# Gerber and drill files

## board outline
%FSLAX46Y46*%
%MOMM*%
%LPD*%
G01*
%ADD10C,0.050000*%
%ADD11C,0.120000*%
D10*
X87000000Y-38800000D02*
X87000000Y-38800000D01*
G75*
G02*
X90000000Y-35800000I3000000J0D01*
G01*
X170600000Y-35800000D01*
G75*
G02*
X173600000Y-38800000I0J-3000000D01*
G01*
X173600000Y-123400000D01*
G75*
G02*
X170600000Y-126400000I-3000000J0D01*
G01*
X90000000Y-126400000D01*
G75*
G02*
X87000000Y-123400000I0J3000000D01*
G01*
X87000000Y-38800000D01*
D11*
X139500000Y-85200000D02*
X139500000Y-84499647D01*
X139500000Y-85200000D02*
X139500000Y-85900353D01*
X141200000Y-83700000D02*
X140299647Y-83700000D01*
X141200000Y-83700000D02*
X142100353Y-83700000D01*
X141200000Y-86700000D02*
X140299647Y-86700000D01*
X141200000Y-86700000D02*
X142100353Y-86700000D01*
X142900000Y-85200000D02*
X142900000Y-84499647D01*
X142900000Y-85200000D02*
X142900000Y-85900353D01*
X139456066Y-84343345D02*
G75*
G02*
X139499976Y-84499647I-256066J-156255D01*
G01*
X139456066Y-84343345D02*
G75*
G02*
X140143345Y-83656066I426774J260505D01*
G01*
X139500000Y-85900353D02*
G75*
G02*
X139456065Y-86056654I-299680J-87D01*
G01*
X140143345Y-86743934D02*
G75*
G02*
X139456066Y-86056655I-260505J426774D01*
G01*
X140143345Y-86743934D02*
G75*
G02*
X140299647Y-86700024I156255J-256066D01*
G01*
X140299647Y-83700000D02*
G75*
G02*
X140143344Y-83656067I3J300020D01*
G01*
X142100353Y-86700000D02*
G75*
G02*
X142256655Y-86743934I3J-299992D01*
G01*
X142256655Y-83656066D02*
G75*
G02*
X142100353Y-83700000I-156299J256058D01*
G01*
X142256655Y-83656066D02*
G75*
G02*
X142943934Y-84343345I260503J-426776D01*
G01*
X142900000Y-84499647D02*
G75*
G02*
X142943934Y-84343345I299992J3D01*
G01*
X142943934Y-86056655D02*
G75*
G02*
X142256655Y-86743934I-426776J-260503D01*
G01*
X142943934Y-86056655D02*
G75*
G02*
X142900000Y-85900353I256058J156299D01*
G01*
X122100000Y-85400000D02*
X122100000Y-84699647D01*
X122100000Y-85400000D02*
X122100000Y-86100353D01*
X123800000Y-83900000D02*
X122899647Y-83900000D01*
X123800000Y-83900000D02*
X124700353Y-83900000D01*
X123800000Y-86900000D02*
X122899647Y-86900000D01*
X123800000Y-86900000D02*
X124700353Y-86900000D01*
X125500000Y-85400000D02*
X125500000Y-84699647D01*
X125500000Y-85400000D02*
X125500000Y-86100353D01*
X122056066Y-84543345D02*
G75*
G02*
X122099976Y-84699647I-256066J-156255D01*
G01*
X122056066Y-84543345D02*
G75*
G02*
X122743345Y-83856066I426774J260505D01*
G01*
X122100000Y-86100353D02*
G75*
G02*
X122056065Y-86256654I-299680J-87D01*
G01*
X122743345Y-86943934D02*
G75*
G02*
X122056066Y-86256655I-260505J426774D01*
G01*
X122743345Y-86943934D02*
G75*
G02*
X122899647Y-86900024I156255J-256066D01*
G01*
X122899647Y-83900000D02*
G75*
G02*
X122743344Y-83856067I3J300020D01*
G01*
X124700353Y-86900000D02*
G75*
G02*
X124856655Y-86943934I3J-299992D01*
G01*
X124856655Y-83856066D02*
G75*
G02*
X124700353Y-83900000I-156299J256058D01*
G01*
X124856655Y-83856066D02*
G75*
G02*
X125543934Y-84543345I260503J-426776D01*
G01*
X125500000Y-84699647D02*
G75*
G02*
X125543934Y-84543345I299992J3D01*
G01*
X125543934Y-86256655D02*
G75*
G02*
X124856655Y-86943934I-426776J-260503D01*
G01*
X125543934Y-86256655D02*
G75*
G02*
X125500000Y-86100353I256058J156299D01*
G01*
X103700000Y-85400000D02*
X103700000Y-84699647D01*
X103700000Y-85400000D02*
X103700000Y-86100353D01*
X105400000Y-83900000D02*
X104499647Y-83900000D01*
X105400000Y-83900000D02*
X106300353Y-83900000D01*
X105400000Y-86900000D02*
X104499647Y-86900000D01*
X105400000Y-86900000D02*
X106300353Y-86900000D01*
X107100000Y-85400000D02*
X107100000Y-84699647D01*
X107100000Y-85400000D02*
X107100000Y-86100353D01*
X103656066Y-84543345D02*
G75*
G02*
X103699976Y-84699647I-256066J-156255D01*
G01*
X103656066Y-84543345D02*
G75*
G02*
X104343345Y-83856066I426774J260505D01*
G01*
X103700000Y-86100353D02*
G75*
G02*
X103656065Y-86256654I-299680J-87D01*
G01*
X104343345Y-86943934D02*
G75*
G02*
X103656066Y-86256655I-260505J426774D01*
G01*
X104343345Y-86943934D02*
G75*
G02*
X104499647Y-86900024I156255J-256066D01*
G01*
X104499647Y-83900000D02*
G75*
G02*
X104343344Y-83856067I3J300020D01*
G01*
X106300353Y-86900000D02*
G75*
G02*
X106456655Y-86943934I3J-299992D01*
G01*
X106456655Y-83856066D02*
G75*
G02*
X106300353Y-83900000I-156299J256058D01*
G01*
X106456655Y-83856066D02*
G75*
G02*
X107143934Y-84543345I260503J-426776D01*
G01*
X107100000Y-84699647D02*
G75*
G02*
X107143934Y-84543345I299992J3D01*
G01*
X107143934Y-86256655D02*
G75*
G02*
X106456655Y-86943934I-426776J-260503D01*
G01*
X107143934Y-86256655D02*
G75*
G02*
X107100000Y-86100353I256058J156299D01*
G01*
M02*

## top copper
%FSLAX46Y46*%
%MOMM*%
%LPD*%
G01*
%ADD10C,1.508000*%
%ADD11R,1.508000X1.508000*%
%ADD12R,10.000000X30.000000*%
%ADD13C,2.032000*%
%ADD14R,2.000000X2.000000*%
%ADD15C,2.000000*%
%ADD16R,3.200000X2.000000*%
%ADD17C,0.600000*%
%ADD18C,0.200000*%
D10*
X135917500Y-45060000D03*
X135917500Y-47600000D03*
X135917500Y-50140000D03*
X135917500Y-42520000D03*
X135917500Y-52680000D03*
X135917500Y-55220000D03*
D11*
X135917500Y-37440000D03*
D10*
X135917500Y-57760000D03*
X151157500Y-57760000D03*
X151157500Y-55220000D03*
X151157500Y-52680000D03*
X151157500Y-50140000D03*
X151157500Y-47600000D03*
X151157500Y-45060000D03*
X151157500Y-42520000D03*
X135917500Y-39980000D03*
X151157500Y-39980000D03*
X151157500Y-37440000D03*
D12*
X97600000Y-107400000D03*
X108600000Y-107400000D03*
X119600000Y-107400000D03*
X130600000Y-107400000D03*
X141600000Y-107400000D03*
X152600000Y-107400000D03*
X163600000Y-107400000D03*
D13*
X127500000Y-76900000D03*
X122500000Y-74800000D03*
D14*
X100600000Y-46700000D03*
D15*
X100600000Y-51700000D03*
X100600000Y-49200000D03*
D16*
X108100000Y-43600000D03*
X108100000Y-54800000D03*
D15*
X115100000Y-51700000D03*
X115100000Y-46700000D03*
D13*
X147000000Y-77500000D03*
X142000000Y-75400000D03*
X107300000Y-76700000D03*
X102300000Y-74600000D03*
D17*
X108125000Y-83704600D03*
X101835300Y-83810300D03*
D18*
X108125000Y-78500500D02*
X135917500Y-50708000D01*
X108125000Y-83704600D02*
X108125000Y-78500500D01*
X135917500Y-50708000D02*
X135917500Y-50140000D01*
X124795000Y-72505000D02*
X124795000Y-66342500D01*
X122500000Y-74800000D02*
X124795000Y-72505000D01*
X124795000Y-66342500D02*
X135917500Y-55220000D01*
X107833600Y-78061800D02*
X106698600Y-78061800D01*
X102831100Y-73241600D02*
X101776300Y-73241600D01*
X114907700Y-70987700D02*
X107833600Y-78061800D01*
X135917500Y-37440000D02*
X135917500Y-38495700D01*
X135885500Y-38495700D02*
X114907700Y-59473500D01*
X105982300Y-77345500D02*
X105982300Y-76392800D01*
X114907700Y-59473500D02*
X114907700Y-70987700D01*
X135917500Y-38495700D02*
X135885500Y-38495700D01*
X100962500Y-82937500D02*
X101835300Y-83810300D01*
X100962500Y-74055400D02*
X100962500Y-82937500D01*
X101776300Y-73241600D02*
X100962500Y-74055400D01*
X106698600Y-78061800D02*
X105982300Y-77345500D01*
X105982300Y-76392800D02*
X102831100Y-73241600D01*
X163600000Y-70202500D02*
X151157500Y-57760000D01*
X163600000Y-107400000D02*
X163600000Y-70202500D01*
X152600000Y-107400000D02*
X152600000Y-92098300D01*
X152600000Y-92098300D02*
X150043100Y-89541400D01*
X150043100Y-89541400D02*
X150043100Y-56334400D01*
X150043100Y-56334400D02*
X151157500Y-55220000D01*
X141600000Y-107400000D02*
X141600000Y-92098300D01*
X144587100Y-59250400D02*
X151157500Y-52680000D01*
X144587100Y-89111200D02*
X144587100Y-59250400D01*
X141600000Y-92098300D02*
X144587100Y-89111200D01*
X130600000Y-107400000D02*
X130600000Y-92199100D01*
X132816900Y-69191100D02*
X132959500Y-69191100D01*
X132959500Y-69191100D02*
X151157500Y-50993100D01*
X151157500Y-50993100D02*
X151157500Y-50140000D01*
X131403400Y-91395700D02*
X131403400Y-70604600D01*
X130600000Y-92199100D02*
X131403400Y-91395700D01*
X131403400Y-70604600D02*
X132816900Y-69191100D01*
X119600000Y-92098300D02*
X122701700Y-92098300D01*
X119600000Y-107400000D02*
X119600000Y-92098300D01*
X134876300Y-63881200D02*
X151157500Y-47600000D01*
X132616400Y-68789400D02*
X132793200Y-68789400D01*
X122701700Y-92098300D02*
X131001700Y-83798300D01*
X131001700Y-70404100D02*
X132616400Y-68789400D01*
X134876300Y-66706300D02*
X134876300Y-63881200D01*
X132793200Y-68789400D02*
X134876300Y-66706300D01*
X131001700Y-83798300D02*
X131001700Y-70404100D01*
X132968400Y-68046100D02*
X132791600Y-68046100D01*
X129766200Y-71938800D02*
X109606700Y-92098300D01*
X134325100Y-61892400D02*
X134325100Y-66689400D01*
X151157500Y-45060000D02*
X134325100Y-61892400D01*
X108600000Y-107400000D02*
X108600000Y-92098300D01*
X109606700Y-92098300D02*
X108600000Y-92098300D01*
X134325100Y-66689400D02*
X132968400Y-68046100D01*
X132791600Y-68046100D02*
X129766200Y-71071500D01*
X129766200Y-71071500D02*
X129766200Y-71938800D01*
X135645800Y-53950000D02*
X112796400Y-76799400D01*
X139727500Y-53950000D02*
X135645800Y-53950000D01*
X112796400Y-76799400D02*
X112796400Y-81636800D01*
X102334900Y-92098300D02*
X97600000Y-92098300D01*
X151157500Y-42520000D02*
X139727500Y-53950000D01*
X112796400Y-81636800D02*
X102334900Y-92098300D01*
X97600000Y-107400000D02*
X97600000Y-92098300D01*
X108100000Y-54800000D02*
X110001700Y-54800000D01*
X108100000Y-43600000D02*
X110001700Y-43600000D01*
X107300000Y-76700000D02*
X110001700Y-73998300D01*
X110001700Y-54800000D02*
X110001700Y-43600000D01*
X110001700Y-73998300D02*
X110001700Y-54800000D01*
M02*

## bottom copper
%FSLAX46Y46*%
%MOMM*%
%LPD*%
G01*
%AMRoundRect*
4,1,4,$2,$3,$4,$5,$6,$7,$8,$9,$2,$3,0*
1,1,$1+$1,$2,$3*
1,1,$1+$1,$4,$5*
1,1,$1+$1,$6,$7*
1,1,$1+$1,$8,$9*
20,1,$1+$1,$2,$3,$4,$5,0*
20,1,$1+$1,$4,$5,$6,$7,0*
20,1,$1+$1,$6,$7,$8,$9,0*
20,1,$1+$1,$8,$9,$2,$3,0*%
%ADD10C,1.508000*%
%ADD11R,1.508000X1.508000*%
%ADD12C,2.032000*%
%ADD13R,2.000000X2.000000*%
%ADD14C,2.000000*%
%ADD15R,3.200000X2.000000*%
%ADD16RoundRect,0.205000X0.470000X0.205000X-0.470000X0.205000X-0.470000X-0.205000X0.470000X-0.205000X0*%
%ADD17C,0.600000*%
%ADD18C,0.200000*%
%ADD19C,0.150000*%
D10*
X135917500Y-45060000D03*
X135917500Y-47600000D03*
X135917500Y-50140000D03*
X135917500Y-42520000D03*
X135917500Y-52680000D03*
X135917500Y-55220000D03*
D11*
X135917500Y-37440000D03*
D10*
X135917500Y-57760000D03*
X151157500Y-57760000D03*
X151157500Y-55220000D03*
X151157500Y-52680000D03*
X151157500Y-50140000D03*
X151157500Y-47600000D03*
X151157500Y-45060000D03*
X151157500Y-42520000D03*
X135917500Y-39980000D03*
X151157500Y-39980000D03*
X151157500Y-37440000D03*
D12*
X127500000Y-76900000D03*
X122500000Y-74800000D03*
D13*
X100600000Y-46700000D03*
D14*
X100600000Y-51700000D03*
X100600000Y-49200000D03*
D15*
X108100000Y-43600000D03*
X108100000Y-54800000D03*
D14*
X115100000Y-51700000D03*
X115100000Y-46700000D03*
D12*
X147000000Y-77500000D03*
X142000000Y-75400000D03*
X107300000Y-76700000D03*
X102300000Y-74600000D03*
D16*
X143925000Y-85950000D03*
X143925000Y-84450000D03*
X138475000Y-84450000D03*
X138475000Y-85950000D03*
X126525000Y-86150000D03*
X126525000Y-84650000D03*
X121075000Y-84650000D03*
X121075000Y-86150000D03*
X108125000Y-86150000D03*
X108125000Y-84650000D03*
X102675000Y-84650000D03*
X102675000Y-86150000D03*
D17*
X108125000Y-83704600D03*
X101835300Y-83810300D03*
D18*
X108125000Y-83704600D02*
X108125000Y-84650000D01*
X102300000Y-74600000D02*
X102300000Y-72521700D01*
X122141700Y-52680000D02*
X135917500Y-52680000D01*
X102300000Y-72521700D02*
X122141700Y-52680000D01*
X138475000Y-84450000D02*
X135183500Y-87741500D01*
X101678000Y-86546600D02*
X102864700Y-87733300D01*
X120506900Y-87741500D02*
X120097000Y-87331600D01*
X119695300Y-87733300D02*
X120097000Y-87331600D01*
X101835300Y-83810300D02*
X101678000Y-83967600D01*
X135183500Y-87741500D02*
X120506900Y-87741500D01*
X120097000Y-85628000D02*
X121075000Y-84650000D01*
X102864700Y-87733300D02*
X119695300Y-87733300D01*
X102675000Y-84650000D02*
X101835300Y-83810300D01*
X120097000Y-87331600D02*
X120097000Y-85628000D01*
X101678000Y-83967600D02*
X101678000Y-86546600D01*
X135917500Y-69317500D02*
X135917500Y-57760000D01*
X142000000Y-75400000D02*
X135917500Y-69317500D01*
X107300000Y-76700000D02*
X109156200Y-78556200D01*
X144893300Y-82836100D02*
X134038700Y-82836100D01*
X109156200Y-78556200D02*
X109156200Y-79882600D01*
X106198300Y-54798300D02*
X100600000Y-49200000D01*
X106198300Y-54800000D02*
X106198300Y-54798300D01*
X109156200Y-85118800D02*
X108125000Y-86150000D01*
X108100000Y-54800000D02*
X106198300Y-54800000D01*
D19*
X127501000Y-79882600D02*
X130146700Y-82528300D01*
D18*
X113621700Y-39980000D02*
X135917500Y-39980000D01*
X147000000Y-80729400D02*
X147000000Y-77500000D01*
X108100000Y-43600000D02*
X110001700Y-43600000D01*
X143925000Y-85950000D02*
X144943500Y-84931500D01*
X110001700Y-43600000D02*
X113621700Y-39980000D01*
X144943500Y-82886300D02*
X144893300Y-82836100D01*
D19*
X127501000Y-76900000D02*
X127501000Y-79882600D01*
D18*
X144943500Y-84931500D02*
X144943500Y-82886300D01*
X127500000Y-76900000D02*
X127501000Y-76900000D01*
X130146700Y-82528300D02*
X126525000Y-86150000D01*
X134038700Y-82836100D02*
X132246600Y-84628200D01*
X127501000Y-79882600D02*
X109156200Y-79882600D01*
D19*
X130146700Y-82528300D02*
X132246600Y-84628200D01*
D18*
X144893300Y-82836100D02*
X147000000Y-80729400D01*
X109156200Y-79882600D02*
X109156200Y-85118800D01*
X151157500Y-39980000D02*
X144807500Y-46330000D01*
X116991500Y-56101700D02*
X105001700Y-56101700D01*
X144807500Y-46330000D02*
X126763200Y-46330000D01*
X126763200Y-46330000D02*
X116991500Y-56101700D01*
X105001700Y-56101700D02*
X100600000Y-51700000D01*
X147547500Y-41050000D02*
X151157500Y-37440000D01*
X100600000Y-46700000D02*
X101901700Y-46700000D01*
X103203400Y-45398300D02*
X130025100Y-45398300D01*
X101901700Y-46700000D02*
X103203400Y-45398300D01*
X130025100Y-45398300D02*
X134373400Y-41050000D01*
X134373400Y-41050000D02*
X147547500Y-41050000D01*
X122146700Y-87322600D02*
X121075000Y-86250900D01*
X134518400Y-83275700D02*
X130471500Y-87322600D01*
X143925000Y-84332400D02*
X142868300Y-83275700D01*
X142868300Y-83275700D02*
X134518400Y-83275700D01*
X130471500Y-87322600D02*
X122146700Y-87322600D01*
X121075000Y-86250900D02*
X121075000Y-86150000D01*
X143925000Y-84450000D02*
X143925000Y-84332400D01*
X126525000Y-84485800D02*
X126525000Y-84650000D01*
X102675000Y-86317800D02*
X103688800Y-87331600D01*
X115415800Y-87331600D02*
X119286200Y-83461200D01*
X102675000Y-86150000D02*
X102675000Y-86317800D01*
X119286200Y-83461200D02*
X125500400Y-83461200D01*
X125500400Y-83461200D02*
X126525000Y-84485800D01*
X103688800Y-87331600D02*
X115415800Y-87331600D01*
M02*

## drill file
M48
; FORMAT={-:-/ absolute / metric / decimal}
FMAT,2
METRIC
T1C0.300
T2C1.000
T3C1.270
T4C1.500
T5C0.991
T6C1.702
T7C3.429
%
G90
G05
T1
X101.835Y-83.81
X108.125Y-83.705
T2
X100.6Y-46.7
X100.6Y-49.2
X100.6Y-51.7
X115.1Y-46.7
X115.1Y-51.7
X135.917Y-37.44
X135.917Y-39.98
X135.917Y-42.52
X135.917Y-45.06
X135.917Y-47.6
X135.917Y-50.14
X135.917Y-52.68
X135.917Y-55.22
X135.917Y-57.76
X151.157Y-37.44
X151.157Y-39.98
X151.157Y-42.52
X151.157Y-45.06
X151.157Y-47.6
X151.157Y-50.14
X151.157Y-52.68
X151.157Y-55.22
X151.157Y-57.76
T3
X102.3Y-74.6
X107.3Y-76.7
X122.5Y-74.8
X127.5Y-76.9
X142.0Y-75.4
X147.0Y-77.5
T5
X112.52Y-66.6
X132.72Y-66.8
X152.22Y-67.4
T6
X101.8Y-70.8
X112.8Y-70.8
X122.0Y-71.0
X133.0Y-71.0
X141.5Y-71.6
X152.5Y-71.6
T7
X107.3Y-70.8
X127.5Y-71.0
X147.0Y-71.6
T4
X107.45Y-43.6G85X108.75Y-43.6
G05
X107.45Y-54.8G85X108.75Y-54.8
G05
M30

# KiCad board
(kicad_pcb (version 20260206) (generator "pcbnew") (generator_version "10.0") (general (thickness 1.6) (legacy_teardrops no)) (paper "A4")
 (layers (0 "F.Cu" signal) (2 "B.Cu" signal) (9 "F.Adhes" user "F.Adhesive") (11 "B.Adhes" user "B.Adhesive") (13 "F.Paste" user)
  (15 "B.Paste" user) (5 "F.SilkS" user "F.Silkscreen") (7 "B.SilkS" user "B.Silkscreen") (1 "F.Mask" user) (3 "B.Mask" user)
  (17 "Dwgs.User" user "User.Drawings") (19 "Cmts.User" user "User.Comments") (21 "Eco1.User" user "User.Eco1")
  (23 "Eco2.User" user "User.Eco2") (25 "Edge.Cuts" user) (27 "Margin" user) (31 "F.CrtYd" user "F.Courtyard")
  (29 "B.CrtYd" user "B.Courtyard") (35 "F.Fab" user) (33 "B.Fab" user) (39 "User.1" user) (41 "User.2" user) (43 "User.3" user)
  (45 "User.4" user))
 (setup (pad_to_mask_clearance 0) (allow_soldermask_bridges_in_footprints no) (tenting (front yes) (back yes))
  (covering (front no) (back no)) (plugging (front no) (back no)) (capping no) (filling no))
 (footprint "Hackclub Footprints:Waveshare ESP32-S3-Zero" (layer "F.Cu") (at 143.5375 47.6)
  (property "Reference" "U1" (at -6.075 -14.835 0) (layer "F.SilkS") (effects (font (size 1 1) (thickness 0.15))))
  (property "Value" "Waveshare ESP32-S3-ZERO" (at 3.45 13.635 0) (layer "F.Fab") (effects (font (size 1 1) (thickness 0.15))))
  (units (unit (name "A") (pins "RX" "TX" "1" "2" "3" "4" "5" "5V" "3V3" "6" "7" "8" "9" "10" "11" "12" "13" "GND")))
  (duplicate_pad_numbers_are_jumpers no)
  (pad "1" thru_hole circle (at -7.62 -2.54) (size 1.508 1.508) (drill 1) (layers "*.Cu" "*.Mask") (remove_unused_layers no)
   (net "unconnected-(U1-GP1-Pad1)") (solder_mask_margin 0.102))
  (pad "2" thru_hole circle (at -7.62 0) (size 1.508 1.508) (drill 1) (layers "*.Cu" "*.Mask") (remove_unused_layers no)
   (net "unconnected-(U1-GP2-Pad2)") (solder_mask_margin 0.102))
  (pad "3" thru_hole circle (at -7.62 2.54) (size 1.508 1.508) (drill 1) (layers "*.Cu" "*.Mask") (remove_unused_layers no) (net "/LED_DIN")
   (solder_mask_margin 0.102))
  (pad "3V3" thru_hole circle (at -7.62 -5.08) (size 1.508 1.508) (drill 1) (layers "*.Cu" "*.Mask") (remove_unused_layers no) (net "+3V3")
   (solder_mask_margin 0.102))
  (pad "4" thru_hole circle (at -7.62 5.08) (size 1.508 1.508) (drill 1) (layers "*.Cu" "*.Mask") (remove_unused_layers no) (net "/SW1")
   (solder_mask_margin 0.102))
  (pad "5" thru_hole circle (at -7.62 7.62) (size 1.508 1.508) (drill 1) (layers "*.Cu" "*.Mask") (remove_unused_layers no) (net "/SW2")
   (solder_mask_margin 0.102))
  (pad "5V" thru_hole rect (at -7.62 -10.16) (size 1.508 1.508) (drill 1) (layers "*.Cu" "*.Mask") (remove_unused_layers no) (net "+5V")
   (solder_mask_margin 0.102))
  (pad "6" thru_hole circle (at -7.62 10.16) (size 1.508 1.508) (drill 1) (layers "*.Cu" "*.Mask") (remove_unused_layers no) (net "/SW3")
   (solder_mask_margin 0.102))
  (pad "7" thru_hole circle (at 7.62 10.16) (size 1.508 1.508) (drill 1) (layers "*.Cu" "*.Mask") (remove_unused_layers no) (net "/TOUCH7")
   (solder_mask_margin 0.102))
  (pad "8" thru_hole circle (at 7.62 7.62) (size 1.508 1.508) (drill 1) (layers "*.Cu" "*.Mask") (remove_unused_layers no) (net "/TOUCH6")
   (solder_mask_margin 0.102))
  (pad "9" thru_hole circle (at 7.62 5.08) (size 1.508 1.508) (drill 1) (layers "*.Cu" "*.Mask") (remove_unused_layers no) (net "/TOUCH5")
   (solder_mask_margin 0.102))
  (pad "10" thru_hole circle (at 7.62 2.54) (size 1.508 1.508) (drill 1) (layers "*.Cu" "*.Mask") (remove_unused_layers no) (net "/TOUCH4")
   (solder_mask_margin 0.102))
  (pad "11" thru_hole circle (at 7.62 0) (size 1.508 1.508) (drill 1) (layers "*.Cu" "*.Mask") (remove_unused_layers no) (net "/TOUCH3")
   (solder_mask_margin 0.102))
  (pad "12" thru_hole circle (at 7.62 -2.54) (size 1.508 1.508) (drill 1) (layers "*.Cu" "*.Mask") (remove_unused_layers no) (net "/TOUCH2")
   (solder_mask_margin 0.102))
  (pad "13" thru_hole circle (at 7.62 -5.08) (size 1.508 1.508) (drill 1) (layers "*.Cu" "*.Mask") (remove_unused_layers no) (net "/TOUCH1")
   (solder_mask_margin 0.102))
  (pad "GND" thru_hole circle (at -7.62 -7.62) (size 1.508 1.508) (drill 1) (layers "*.Cu" "*.Mask") (remove_unused_layers no) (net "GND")
   (solder_mask_margin 0.102))
  (pad "RX" thru_hole circle (at 7.62 -7.62) (size 1.508 1.508) (drill 1) (layers "*.Cu" "*.Mask") (remove_unused_layers no) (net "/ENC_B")
   (solder_mask_margin 0.102))
  (pad "TX" thru_hole circle (at 7.62 -10.16) (size 1.508 1.508) (drill 1) (layers "*.Cu" "*.Mask") (remove_unused_layers no) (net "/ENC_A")
   (solder_mask_margin 0.102)))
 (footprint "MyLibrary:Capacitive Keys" (layer "F.Cu") (at 97.6 107.4)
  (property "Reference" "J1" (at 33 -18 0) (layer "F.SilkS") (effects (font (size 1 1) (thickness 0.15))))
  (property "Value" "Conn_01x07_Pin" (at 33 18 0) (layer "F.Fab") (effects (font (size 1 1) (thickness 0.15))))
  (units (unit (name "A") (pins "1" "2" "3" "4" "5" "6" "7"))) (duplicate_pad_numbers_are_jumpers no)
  (pad "1" smd rect (at 0 0) (size 10 30) (layers "F.Cu" "F.Mask") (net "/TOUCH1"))
  (pad "2" smd rect (at 11 0) (size 10 30) (layers "F.Cu" "F.Mask") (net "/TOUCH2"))
  (pad "3" smd rect (at 22 0) (size 10 30) (layers "F.Cu" "F.Mask") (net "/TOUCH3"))
  (pad "4" smd rect (at 33 0) (size 10 30) (layers "F.Cu" "F.Mask") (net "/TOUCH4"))
  (pad "5" smd rect (at 44 0) (size 10 30) (layers "F.Cu" "F.Mask") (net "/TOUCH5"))
  (pad "6" smd rect (at 55 0) (size 10 30) (layers "F.Cu" "F.Mask") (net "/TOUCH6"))
  (pad "7" smd rect (at 66 0) (size 10 30) (layers "F.Cu" "F.Mask") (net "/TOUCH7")))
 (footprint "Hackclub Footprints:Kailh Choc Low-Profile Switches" (layer "F.Cu") (at 127.5 71)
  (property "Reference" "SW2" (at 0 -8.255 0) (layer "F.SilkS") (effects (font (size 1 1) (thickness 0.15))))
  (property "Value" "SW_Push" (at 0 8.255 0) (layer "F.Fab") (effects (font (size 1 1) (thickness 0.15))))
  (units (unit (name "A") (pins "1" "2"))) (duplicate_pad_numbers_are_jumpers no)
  (pad "" np_thru_hole circle (at -5.5 0) (size 1.7018 1.7018) (drill 1.7018) (layers "*.Cu" "*.Mask"))
  (pad "" np_thru_hole circle (at 0 0) (size 3.429 3.429) (drill 3.429) (layers "*.Cu" "*.Mask"))
  (pad "" np_thru_hole circle (at 5.22 -4.2) (size 0.9906 0.9906) (drill 0.9906) (layers "*.Cu" "*.Mask"))
  (pad "" np_thru_hole circle (at 5.5 0) (size 1.7018 1.7018) (drill 1.7018) (layers "*.Cu" "*.Mask"))
  (pad "1" thru_hole circle (at 0 5.9) (size 2.032 2.032) (drill 1.27) (layers "*.Cu" "*.Mask") (remove_unused_layers no) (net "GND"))
  (pad "2" thru_hole circle (at -5 3.8) (size 2.032 2.032) (drill 1.27) (layers "*.Cu" "*.Mask") (remove_unused_layers no) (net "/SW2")))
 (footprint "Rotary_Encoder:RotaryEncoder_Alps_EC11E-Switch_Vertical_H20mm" (layer "F.Cu") (at 100.6 46.7)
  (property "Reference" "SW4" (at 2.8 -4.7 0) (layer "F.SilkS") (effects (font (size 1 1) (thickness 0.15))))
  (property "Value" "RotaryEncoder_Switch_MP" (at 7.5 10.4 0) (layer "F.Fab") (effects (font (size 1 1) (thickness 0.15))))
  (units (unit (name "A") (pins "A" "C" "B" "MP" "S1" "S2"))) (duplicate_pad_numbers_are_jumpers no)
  (pad "A" thru_hole rect (at 0 0) (size 2 2) (drill 1) (layers "*.Cu" "*.Mask") (remove_unused_layers no) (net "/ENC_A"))
  (pad "B" thru_hole circle (at 0 5) (size 2 2) (drill 1) (layers "*.Cu" "*.Mask") (remove_unused_layers no) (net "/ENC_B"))
  (pad "C" thru_hole circle (at 0 2.5) (size 2 2) (drill 1) (layers "*.Cu" "*.Mask") (remove_unused_layers no) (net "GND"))
  (pad "MP" thru_hole rect (at 7.5 -3.1) (size 3.2 2) (drill oval 2.8 1.5) (layers "*.Cu" "*.Mask") (remove_unused_layers no) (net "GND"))
  (pad "MP" thru_hole rect (at 7.5 8.1) (size 3.2 2) (drill oval 2.8 1.5) (layers "*.Cu" "*.Mask") (remove_unused_layers no) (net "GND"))
  (pad "S1" thru_hole circle (at 14.5 5) (size 2 2) (drill 1) (layers "*.Cu" "*.Mask") (remove_unused_layers no)
   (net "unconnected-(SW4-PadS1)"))
  (pad "S2" thru_hole circle (at 14.5 0) (size 2 2) (drill 1) (layers "*.Cu" "*.Mask") (remove_unused_layers no)
   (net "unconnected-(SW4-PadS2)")))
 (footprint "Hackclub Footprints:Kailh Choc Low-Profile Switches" (layer "F.Cu") (at 147 71.6)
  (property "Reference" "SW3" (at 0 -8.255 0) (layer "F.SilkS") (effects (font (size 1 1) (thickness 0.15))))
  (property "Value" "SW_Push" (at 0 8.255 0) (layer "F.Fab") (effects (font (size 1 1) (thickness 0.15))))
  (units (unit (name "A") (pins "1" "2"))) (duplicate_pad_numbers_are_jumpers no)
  (pad "" np_thru_hole circle (at -5.5 0) (size 1.7018 1.7018) (drill 1.7018) (layers "*.Cu" "*.Mask"))
  (pad "" np_thru_hole circle (at 0 0) (size 3.429 3.429) (drill 3.429) (layers "*.Cu" "*.Mask"))
  (pad "" np_thru_hole circle (at 5.22 -4.2) (size 0.9906 0.9906) (drill 0.9906) (layers "*.Cu" "*.Mask"))
  (pad "" np_thru_hole circle (at 5.5 0) (size 1.7018 1.7018) (drill 1.7018) (layers "*.Cu" "*.Mask"))
  (pad "1" thru_hole circle (at 0 5.9) (size 2.032 2.032) (drill 1.27) (layers "*.Cu" "*.Mask") (remove_unused_layers no) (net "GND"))
  (pad "2" thru_hole circle (at -5 3.8) (size 2.032 2.032) (drill 1.27) (layers "*.Cu" "*.Mask") (remove_unused_layers no) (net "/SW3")))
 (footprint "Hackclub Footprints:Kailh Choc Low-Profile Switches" (layer "F.Cu") (at 107.3 70.8)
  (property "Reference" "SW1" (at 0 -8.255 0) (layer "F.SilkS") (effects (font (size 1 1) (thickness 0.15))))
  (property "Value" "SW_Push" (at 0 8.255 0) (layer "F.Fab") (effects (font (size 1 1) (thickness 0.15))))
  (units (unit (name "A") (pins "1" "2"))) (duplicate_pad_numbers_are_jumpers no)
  (pad "" np_thru_hole circle (at -5.5 0) (size 1.7018 1.7018) (drill 1.7018) (layers "*.Cu" "*.Mask"))
  (pad "" np_thru_hole circle (at 0 0) (size 3.429 3.429) (drill 3.429) (layers "*.Cu" "*.Mask"))
  (pad "" np_thru_hole circle (at 5.22 -4.2) (size 0.9906 0.9906) (drill 0.9906) (layers "*.Cu" "*.Mask"))
  (pad "" np_thru_hole circle (at 5.5 0) (size 1.7018 1.7018) (drill 1.7018) (layers "*.Cu" "*.Mask"))
  (pad "1" thru_hole circle (at 0 5.9) (size 2.032 2.032) (drill 1.27) (layers "*.Cu" "*.Mask") (remove_unused_layers no) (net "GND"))
  (pad "2" thru_hole circle (at -5 3.8) (size 2.032 2.032) (drill 1.27) (layers "*.Cu" "*.Mask") (remove_unused_layers no) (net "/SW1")))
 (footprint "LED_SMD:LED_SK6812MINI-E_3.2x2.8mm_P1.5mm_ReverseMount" (layer "B.Cu") (at 141.2 85.2 180)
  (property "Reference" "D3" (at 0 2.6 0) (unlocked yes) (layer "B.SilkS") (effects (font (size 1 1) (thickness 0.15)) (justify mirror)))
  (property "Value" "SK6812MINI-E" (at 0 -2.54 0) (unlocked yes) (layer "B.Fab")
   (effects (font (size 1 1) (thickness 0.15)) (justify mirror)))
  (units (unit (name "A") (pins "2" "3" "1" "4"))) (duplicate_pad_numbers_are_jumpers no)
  (fp_line (start 1.7 0) (end 1.7 0.700353) (stroke (width 0.12) (type solid)) (layer "Edge.Cuts"))
  (fp_line (start 1.7 0) (end 1.7 -0.700353) (stroke (width 0.12) (type solid)) (layer "Edge.Cuts"))
  (fp_line (start 0 1.5) (end 0.900353 1.5) (stroke (width 0.12) (type solid)) (layer "Edge.Cuts"))
  (fp_line (start 0 1.5) (end -0.900353 1.5) (stroke (width 0.12) (type solid)) (layer "Edge.Cuts"))
  (fp_line (start 0 -1.5) (end 0.900353 -1.5) (stroke (width 0.12) (type solid)) (layer "Edge.Cuts"))
  (fp_line (start 0 -1.5) (end -0.900353 -1.5) (stroke (width 0.12) (type solid)) (layer "Edge.Cuts"))
  (fp_line (start -1.7 0) (end -1.7 0.700353) (stroke (width 0.12) (type solid)) (layer "Edge.Cuts"))
  (fp_line (start -1.7 0) (end -1.7 -0.700353) (stroke (width 0.12) (type solid)) (layer "Edge.Cuts"))
  (fp_arc (start 1.743934 0.856655) (mid 1.711191 0.781533) (end 1.7 0.700353) (stroke (width 0.12) (type solid)) (layer "Edge.Cuts"))
  (fp_arc (start 1.743934 0.856655) (mid 1.670713 1.470713) (end 1.056655 1.543934) (stroke (width 0.12) (type solid)) (layer "Edge.Cuts"))
  (fp_arc (start 1.7 -0.700353) (mid 1.711181 -0.781538) (end 1.743934 -0.856655) (stroke (width 0.12) (type solid)) (layer "Edge.Cuts"))
  (fp_arc (start 1.056655 -1.543934) (mid 1.670711 -1.470711) (end 1.743934 -0.856655) (stroke (width 0.12) (type solid))
   (layer "Edge.Cuts"))
  (fp_arc (start 1.056655 -1.543934) (mid 0.981533 -1.511191) (end 0.900353 -1.5) (stroke (width 0.12) (type solid)) (layer "Edge.Cuts"))
  (fp_arc (start 0.900353 1.5) (mid 0.981532 1.511193) (end 1.056655 1.543934) (stroke (width 0.12) (type solid)) (layer "Edge.Cuts"))
  (fp_arc (start -0.900353 -1.5) (mid -0.981533 -1.511192) (end -1.056655 -1.543934) (stroke (width 0.12) (type solid)) (layer "Edge.Cuts"))
  (fp_arc (start -1.056655 1.543934) (mid -0.981533 1.511192) (end -0.900353 1.5) (stroke (width 0.12) (type solid)) (layer "Edge.Cuts"))
  (fp_arc (start -1.056655 1.543934) (mid -1.670711 1.470711) (end -1.743934 0.856655) (stroke (width 0.12) (type solid))
   (layer "Edge.Cuts"))
  (fp_arc (start -1.7 0.700353) (mid -1.711192 0.781533) (end -1.743934 0.856655) (stroke (width 0.12) (type solid)) (layer "Edge.Cuts"))
  (fp_arc (start -1.743934 -0.856655) (mid -1.670711 -1.470711) (end -1.056655 -1.543934) (stroke (width 0.12) (type solid))
   (layer "Edge.Cuts"))
  (fp_arc (start -1.743934 -0.856655) (mid -1.711192 -0.781533) (end -1.7 -0.700353) (stroke (width 0.12) (type solid)) (layer "Edge.Cuts"))
  (pad "1" smd roundrect (at -2.725 -0.75 180) (size 1.35 0.82) (layers "B.Cu" "B.Mask" "B.Paste") (roundrect_rratio 0.25) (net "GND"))
  (pad "2" smd roundrect (at -2.725 0.75 180) (size 1.35 0.82) (layers "B.Cu" "B.Mask" "B.Paste") (roundrect_rratio 0.25) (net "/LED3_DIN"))
  (pad "3" smd roundrect (at 2.725 0.75 180) (size 1.35 0.82) (layers "B.Cu" "B.Mask" "B.Paste") (roundrect_rratio 0.25) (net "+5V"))
  (pad "4" smd roundrect (at 2.725 -0.75 180) (size 1.35 0.82) (layers "B.Cu" "B.Mask" "B.Paste") (roundrect_rratio 0.25)
   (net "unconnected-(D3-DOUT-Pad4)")))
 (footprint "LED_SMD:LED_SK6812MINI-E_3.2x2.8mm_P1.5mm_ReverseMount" (layer "B.Cu") (at 123.8 85.4 180)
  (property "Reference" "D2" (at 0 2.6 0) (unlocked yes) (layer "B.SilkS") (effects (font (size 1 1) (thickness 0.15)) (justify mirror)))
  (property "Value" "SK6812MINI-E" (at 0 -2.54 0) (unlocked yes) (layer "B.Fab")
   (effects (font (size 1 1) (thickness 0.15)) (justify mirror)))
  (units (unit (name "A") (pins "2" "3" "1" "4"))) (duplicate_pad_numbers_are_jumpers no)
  (fp_line (start 1.7 0) (end 1.7 0.700353) (stroke (width 0.12) (type solid)) (layer "Edge.Cuts"))
  (fp_line (start 1.7 0) (end 1.7 -0.700353) (stroke (width 0.12) (type solid)) (layer "Edge.Cuts"))
  (fp_line (start 0 1.5) (end 0.900353 1.5) (stroke (width 0.12) (type solid)) (layer "Edge.Cuts"))
  (fp_line (start 0 1.5) (end -0.900353 1.5) (stroke (width 0.12) (type solid)) (layer "Edge.Cuts"))
  (fp_line (start 0 -1.5) (end 0.900353 -1.5) (stroke (width 0.12) (type solid)) (layer "Edge.Cuts"))
  (fp_line (start 0 -1.5) (end -0.900353 -1.5) (stroke (width 0.12) (type solid)) (layer "Edge.Cuts"))
  (fp_line (start -1.7 0) (end -1.7 0.700353) (stroke (width 0.12) (type solid)) (layer "Edge.Cuts"))
  (fp_line (start -1.7 0) (end -1.7 -0.700353) (stroke (width 0.12) (type solid)) (layer "Edge.Cuts"))
  (fp_arc (start 1.743934 0.856655) (mid 1.711191 0.781533) (end 1.7 0.700353) (stroke (width 0.12) (type solid)) (layer "Edge.Cuts"))
  (fp_arc (start 1.743934 0.856655) (mid 1.670713 1.470713) (end 1.056655 1.543934) (stroke (width 0.12) (type solid)) (layer "Edge.Cuts"))
  (fp_arc (start 1.7 -0.700353) (mid 1.711181 -0.781538) (end 1.743934 -0.856655) (stroke (width 0.12) (type solid)) (layer "Edge.Cuts"))
  (fp_arc (start 1.056655 -1.543934) (mid 1.670711 -1.470711) (end 1.743934 -0.856655) (stroke (width 0.12) (type solid))
   (layer "Edge.Cuts"))
  (fp_arc (start 1.056655 -1.543934) (mid 0.981533 -1.511191) (end 0.900353 -1.5) (stroke (width 0.12) (type solid)) (layer "Edge.Cuts"))
  (fp_arc (start 0.900353 1.5) (mid 0.981532 1.511193) (end 1.056655 1.543934) (stroke (width 0.12) (type solid)) (layer "Edge.Cuts"))
  (fp_arc (start -0.900353 -1.5) (mid -0.981533 -1.511192) (end -1.056655 -1.543934) (stroke (width 0.12) (type solid)) (layer "Edge.Cuts"))
  (fp_arc (start -1.056655 1.543934) (mid -0.981533 1.511192) (end -0.900353 1.5) (stroke (width 0.12) (type solid)) (layer "Edge.Cuts"))
  (fp_arc (start -1.056655 1.543934) (mid -1.670711 1.470711) (end -1.743934 0.856655) (stroke (width 0.12) (type solid))
   (layer "Edge.Cuts"))
  (fp_arc (start -1.7 0.700353) (mid -1.711192 0.781533) (end -1.743934 0.856655) (stroke (width 0.12) (type solid)) (layer "Edge.Cuts"))
  (fp_arc (start -1.743934 -0.856655) (mid -1.670711 -1.470711) (end -1.056655 -1.543934) (stroke (width 0.12) (type solid))
   (layer "Edge.Cuts"))
  (fp_arc (start -1.743934 -0.856655) (mid -1.711192 -0.781533) (end -1.7 -0.700353) (stroke (width 0.12) (type solid)) (layer "Edge.Cuts"))
  (pad "1" smd roundrect (at -2.725 -0.75 180) (size 1.35 0.82) (layers "B.Cu" "B.Mask" "B.Paste") (roundrect_rratio 0.25) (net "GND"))
  (pad "2" smd roundrect (at -2.725 0.75 180) (size 1.35 0.82) (layers "B.Cu" "B.Mask" "B.Paste") (roundrect_rratio 0.25) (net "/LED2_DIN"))
  (pad "3" smd roundrect (at 2.725 0.75 180) (size 1.35 0.82) (layers "B.Cu" "B.Mask" "B.Paste") (roundrect_rratio 0.25) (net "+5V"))
  (pad "4" smd roundrect (at 2.725 -0.75 180) (size 1.35 0.82) (layers "B.Cu" "B.Mask" "B.Paste") (roundrect_rratio 0.25) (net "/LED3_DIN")))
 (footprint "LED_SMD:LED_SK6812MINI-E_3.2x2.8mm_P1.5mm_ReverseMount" (layer "B.Cu") (at 105.4 85.4 180)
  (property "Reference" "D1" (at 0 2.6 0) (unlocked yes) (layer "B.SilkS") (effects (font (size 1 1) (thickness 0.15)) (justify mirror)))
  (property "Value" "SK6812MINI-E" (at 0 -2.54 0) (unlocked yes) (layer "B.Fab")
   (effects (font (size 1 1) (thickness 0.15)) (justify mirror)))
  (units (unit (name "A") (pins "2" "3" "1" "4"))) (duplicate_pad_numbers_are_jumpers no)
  (fp_line (start 1.7 0) (end 1.7 0.700353) (stroke (width 0.12) (type solid)) (layer "Edge.Cuts"))
  (fp_line (start 1.7 0) (end 1.7 -0.700353) (stroke (width 0.12) (type solid)) (layer "Edge.Cuts"))
  (fp_line (start 0 1.5) (end 0.900353 1.5) (stroke (width 0.12) (type solid)) (layer "Edge.Cuts"))
  (fp_line (start 0 1.5) (end -0.900353 1.5) (stroke (width 0.12) (type solid)) (layer "Edge.Cuts"))
  (fp_line (start 0 -1.5) (end 0.900353 -1.5) (stroke (width 0.12) (type solid)) (layer "Edge.Cuts"))
  (fp_line (start 0 -1.5) (end -0.900353 -1.5) (stroke (width 0.12) (type solid)) (layer "Edge.Cuts"))
  (fp_line (start -1.7 0) (end -1.7 0.700353) (stroke (width 0.12) (type solid)) (layer "Edge.Cuts"))
  (fp_line (start -1.7 0) (end -1.7 -0.700353) (stroke (width 0.12) (type solid)) (layer "Edge.Cuts"))
  (fp_arc (start 1.743934 0.856655) (mid 1.711191 0.781533) (end 1.7 0.700353) (stroke (width 0.12) (type solid)) (layer "Edge.Cuts"))
  (fp_arc (start 1.743934 0.856655) (mid 1.670713 1.470713) (end 1.056655 1.543934) (stroke (width 0.12) (type solid)) (layer "Edge.Cuts"))
  (fp_arc (start 1.7 -0.700353) (mid 1.711181 -0.781538) (end 1.743934 -0.856655) (stroke (width 0.12) (type solid)) (layer "Edge.Cuts"))
  (fp_arc (start 1.056655 -1.543934) (mid 1.670711 -1.470711) (end 1.743934 -0.856655) (stroke (width 0.12) (type solid))
   (layer "Edge.Cuts"))
  (fp_arc (start 1.056655 -1.543934) (mid 0.981533 -1.511191) (end 0.900353 -1.5) (stroke (width 0.12) (type solid)) (layer "Edge.Cuts"))
  (fp_arc (start 0.900353 1.5) (mid 0.981532 1.511193) (end 1.056655 1.543934) (stroke (width 0.12) (type solid)) (layer "Edge.Cuts"))
  (fp_arc (start -0.900353 -1.5) (mid -0.981533 -1.511192) (end -1.056655 -1.543934) (stroke (width 0.12) (type solid)) (layer "Edge.Cuts"))
  (fp_arc (start -1.056655 1.543934) (mid -0.981533 1.511192) (end -0.900353 1.5) (stroke (width 0.12) (type solid)) (layer "Edge.Cuts"))
  (fp_arc (start -1.056655 1.543934) (mid -1.670711 1.470711) (end -1.743934 0.856655) (stroke (width 0.12) (type solid))
   (layer "Edge.Cuts"))
  (fp_arc (start -1.7 0.700353) (mid -1.711192 0.781533) (end -1.743934 0.856655) (stroke (width 0.12) (type solid)) (layer "Edge.Cuts"))
  (fp_arc (start -1.743934 -0.856655) (mid -1.670711 -1.470711) (end -1.056655 -1.543934) (stroke (width 0.12) (type solid))
   (layer "Edge.Cuts"))
  (fp_arc (start -1.743934 -0.856655) (mid -1.711192 -0.781533) (end -1.7 -0.700353) (stroke (width 0.12) (type solid)) (layer "Edge.Cuts"))
  (pad "1" smd roundrect (at -2.725 -0.75 180) (size 1.35 0.82) (layers "B.Cu" "B.Mask" "B.Paste") (roundrect_rratio 0.25) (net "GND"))
  (pad "2" smd roundrect (at -2.725 0.75 180) (size 1.35 0.82) (layers "B.Cu" "B.Mask" "B.Paste") (roundrect_rratio 0.25) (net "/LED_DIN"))
  (pad "3" smd roundrect (at 2.725 0.75 180) (size 1.35 0.82) (layers "B.Cu" "B.Mask" "B.Paste") (roundrect_rratio 0.25) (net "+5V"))
  (pad "4" smd roundrect (at 2.725 -0.75 180) (size 1.35 0.82) (layers "B.Cu" "B.Mask" "B.Paste") (roundrect_rratio 0.25) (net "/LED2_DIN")))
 (gr_rect (start 87 35.8) (end 173.6 126.4) (radius 3) (stroke (width 0.05) (type solid)) (fill no) (layer "Edge.Cuts"))
 (segment (start 108.125 78.5005) (end 135.9175 50.708) (width 0.2) (layer "F.Cu") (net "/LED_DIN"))
 (segment (start 108.125 83.7046) (end 108.125 78.5005) (width 0.2) (layer "F.Cu") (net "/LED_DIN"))
 (segment (start 135.9175 50.708) (end 135.9175 50.14) (width 0.2) (layer "F.Cu") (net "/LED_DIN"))
 (via (at 108.125 83.7046) (size 0.6) (drill 0.3) (layers "F.Cu" "B.Cu") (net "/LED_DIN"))
 (segment (start 108.125 83.7046) (end 108.125 84.65) (width 0.2) (layer "B.Cu") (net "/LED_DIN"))
 (segment (start 102.3 74.6) (end 102.3 72.5217) (width 0.2) (layer "B.Cu") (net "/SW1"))
 (segment (start 122.1417 52.68) (end 135.9175 52.68) (width 0.2) (layer "B.Cu") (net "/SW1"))
 (segment (start 102.3 72.5217) (end 122.1417 52.68) (width 0.2) (layer "B.Cu") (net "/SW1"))
 (segment (start 124.795 72.505) (end 124.795 66.3425) (width 0.2) (layer "F.Cu") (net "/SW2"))
 (segment (start 122.5 74.8) (end 124.795 72.505) (width 0.2) (layer "F.Cu") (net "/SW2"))
 (segment (start 124.795 66.3425) (end 135.9175 55.22) (width 0.2) (layer "F.Cu") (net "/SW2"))
 (segment (start 107.8336 78.0618) (end 106.6986 78.0618) (width 0.2) (layer "F.Cu") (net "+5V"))
 (segment (start 102.8311 73.2416) (end 101.7763 73.2416) (width 0.2) (layer "F.Cu") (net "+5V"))
 (segment (start 114.9077 70.9877) (end 107.8336 78.0618) (width 0.2) (layer "F.Cu") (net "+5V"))
 (segment (start 135.9175 37.44) (end 135.9175 38.4957) (width 0.2) (layer "F.Cu") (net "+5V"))
 (segment (start 135.8855 38.4957) (end 114.9077 59.4735) (width 0.2) (layer "F.Cu") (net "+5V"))
 (segment (start 105.9823 77.3455) (end 105.9823 76.3928) (width 0.2) (layer "F.Cu") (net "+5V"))
 (segment (start 114.9077 59.4735) (end 114.9077 70.9877) (width 0.2) (layer "F.Cu") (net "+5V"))
 (segment (start 135.9175 38.4957) (end 135.8855 38.4957) (width 0.2) (layer "F.Cu") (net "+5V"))
 (segment (start 100.9625 82.9375) (end 101.8353 83.8103) (width 0.2) (layer "F.Cu") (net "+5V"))
 (segment (start 100.9625 74.0554) (end 100.9625 82.9375) (width 0.2) (layer "F.Cu") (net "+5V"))
 (segment (start 101.7763 73.2416) (end 100.9625 74.0554) (width 0.2) (layer "F.Cu") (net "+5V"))
 (segment (start 106.6986 78.0618) (end 105.9823 77.3455) (width 0.2) (layer "F.Cu") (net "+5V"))
 (segment (start 105.9823 76.3928) (end 102.8311 73.2416) (width 0.2) (layer "F.Cu") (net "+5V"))
 (via (at 101.8353 83.8103) (size 0.6) (drill 0.3) (layers "F.Cu" "B.Cu") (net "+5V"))
 (segment (start 138.475 84.45) (end 135.1835 87.7415) (width 0.2) (layer "B.Cu") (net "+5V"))
 (segment (start 101.678 86.5466) (end 102.8647 87.7333) (width 0.2) (layer "B.Cu") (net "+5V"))
 (segment (start 120.5069 87.7415) (end 120.097 87.3316) (width 0.2) (layer "B.Cu") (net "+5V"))
 (segment (start 119.6953 87.7333) (end 120.097 87.3316) (width 0.2) (layer "B.Cu") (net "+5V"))
 (segment (start 101.8353 83.8103) (end 101.678 83.9676) (width 0.2) (layer "B.Cu") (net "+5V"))
 (segment (start 135.1835 87.7415) (end 120.5069 87.7415) (width 0.2) (layer "B.Cu") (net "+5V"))
 (segment (start 120.097 85.628) (end 121.075 84.65) (width 0.2) (layer "B.Cu") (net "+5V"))
 (segment (start 102.8647 87.7333) (end 119.6953 87.7333) (width 0.2) (layer "B.Cu") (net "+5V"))
 (segment (start 102.675 84.65) (end 101.8353 83.8103) (width 0.2) (layer "B.Cu") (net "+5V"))
 (segment (start 120.097 87.3316) (end 120.097 85.628) (width 0.2) (layer "B.Cu") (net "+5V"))
 (segment (start 101.678 83.9676) (end 101.678 86.5466) (width 0.2) (layer "B.Cu") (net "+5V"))
 (segment (start 135.9175 69.3175) (end 135.9175 57.76) (width 0.2) (layer "B.Cu") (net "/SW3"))
 (segment (start 142 75.4) (end 135.9175 69.3175) (width 0.2) (layer "B.Cu") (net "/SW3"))
 (segment (start 163.6 70.2025) (end 151.1575 57.76) (width 0.2) (layer "F.Cu") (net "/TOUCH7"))
 (segment (start 163.6 107.4) (end 163.6 70.2025) (width 0.2) (layer "F.Cu") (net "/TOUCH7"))
 (segment (start 152.6 107.4) (end 152.6 92.0983) (width 0.2) (layer "F.Cu") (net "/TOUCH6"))
 (segment (start 152.6 92.0983) (end 150.0431 89.5414) (width 0.2) (layer "F.Cu") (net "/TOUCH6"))
 (segment (start 150.0431 89.5414) (end 150.0431 56.3344) (width 0.2) (layer "F.Cu") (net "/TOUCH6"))
 (segment (start 150.0431 56.3344) (end 151.1575 55.22) (width 0.2) (layer "F.Cu") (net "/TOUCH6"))
 (segment (start 141.6 107.4) (end 141.6 92.0983) (width 0.2) (layer "F.Cu") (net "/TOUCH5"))
 (segment (start 144.5871 59.2504) (end 151.1575 52.68) (width 0.2) (layer "F.Cu") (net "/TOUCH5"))
 (segment (start 144.5871 89.1112) (end 144.5871 59.2504) (width 0.2) (layer "F.Cu") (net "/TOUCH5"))
 (segment (start 141.6 92.0983) (end 144.5871 89.1112) (width 0.2) (layer "F.Cu") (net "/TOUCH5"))
 (segment (start 130.6 107.4) (end 130.6 92.1991) (width 0.2) (layer "F.Cu") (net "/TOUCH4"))
 (segment (start 132.8169 69.1911) (end 132.9595 69.1911) (width 0.2) (layer "F.Cu") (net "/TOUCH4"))
 (segment (start 132.9595 69.1911) (end 151.1575 50.9931) (width 0.2) (layer "F.Cu") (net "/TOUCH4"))
 (segment (start 151.1575 50.9931) (end 151.1575 50.14) (width 0.2) (layer "F.Cu") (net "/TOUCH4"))
 (segment (start 131.4034 91.3957) (end 131.4034 70.6046) (width 0.2) (layer "F.Cu") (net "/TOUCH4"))
 (segment (start 130.6 92.1991) (end 131.4034 91.3957) (width 0.2) (layer "F.Cu") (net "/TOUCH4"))
 (segment (start 131.4034 70.6046) (end 132.8169 69.1911) (width 0.2) (layer "F.Cu") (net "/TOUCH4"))
 (segment (start 119.6 92.0983) (end 122.7017 92.0983) (width 0.2) (layer "F.Cu") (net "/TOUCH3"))
 (segment (start 119.6 107.4) (end 119.6 92.0983) (width 0.2) (layer "F.Cu") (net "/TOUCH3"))
 (segment (start 134.8763 63.8812) (end 151.1575 47.6) (width 0.2) (layer "F.Cu") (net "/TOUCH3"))
 (segment (start 132.6164 68.7894) (end 132.7932 68.7894) (width 0.2) (layer "F.Cu") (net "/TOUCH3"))
 (segment (start 122.7017 92.0983) (end 131.0017 83.7983) (width 0.2) (layer "F.Cu") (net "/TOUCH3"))
 (segment (start 131.0017 70.4041) (end 132.6164 68.7894) (width 0.2) (layer "F.Cu") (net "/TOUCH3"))
 (segment (start 134.8763 66.7063) (end 134.8763 63.8812) (width 0.2) (layer "F.Cu") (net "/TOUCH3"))
 (segment (start 132.7932 68.7894) (end 134.8763 66.7063) (width 0.2) (layer "F.Cu") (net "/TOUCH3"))
 (segment (start 131.0017 83.7983) (end 131.0017 70.4041) (width 0.2) (layer "F.Cu") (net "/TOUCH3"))
 (segment (start 132.9684 68.0461) (end 132.7916 68.0461) (width 0.2) (layer "F.Cu") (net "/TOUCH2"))
 (segment (start 129.7662 71.9388) (end 109.6067 92.0983) (width 0.2) (layer "F.Cu") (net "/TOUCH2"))
 (segment (start 134.3251 61.8924) (end 134.3251 66.6894) (width 0.2) (layer "F.Cu") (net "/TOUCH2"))
 (segment (start 151.1575 45.06) (end 134.3251 61.8924) (width 0.2) (layer "F.Cu") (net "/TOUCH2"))
 (segment (start 108.6 107.4) (end 108.6 92.0983) (width 0.2) (layer "F.Cu") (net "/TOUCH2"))
 (segment (start 109.6067 92.0983) (end 108.6 92.0983) (width 0.2) (layer "F.Cu") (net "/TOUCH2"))
 (segment (start 134.3251 66.6894) (end 132.9684 68.0461) (width 0.2) (layer "F.Cu") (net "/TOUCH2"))
 (segment (start 132.7916 68.0461) (end 129.7662 71.0715) (width 0.2) (layer "F.Cu") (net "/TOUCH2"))
 (segment (start 129.7662 71.0715) (end 129.7662 71.9388) (width 0.2) (layer "F.Cu") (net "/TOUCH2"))
 (segment (start 135.6458 53.95) (end 112.7964 76.7994) (width 0.2) (layer "F.Cu") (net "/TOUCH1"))
 (segment (start 139.7275 53.95) (end 135.6458 53.95) (width 0.2) (layer "F.Cu") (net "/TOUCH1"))
 (segment (start 112.7964 76.7994) (end 112.7964 81.6368) (width 0.2) (layer "F.Cu") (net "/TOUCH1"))
 (segment (start 102.3349 92.0983) (end 97.6 92.0983) (width 0.2) (layer "F.Cu") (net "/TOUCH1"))
 (segment (start 151.1575 42.52) (end 139.7275 53.95) (width 0.2) (layer "F.Cu") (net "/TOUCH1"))
 (segment (start 112.7964 81.6368) (end 102.3349 92.0983) (width 0.2) (layer "F.Cu") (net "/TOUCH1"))
 (segment (start 97.6 107.4) (end 97.6 92.0983) (width 0.2) (layer "F.Cu") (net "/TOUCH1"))
 (segment (start 108.1 54.8) (end 110.0017 54.8) (width 0.2) (layer "F.Cu") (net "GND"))
 (segment (start 108.1 43.6) (end 110.0017 43.6) (width 0.2) (layer "F.Cu") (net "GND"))
 (segment (start 107.3 76.7) (end 110.0017 73.9983) (width 0.2) (layer "F.Cu") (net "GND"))
 (segment (start 110.0017 54.8) (end 110.0017 43.6) (width 0.2) (layer "F.Cu") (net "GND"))
 (segment (start 110.0017 73.9983) (end 110.0017 54.8) (width 0.2) (layer "F.Cu") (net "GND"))
 (segment (start 107.3 76.7) (end 109.1562 78.5562) (width 0.2) (layer "B.Cu") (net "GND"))
 (segment (start 144.8933 82.8361) (end 134.0387 82.8361) (width 0.2) (layer "B.Cu") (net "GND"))
 (segment (start 109.1562 78.5562) (end 109.1562 79.8826) (width 0.2) (layer "B.Cu") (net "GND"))
 (segment (start 106.1983 54.7983) (end 100.6 49.2) (width 0.2) (layer "B.Cu") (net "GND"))
 (segment (start 106.1983 54.8) (end 106.1983 54.7983) (width 0.2) (layer "B.Cu") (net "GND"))
 (segment (start 109.1562 85.1188) (end 108.125 86.15) (width 0.2) (layer "B.Cu") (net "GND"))
 (segment (start 108.1 54.8) (end 106.1983 54.8) (width 0.2) (layer "B.Cu") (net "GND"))
 (segment (start 127.501 79.8826) (end 130.1467 82.5283) (width 0.15) (layer "B.Cu") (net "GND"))
 (segment (start 113.6217 39.98) (end 135.9175 39.98) (width 0.2) (layer "B.Cu") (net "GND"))
 (segment (start 147 80.7294) (end 147 77.5) (width 0.2) (layer "B.Cu") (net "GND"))
 (segment (start 108.1 43.6) (end 110.0017 43.6) (width 0.2) (layer "B.Cu") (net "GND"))
 (segment (start 143.925 85.95) (end 144.9435 84.9315) (width 0.2) (layer "B.Cu") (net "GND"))
 (segment (start 110.0017 43.6) (end 113.6217 39.98) (width 0.2) (layer "B.Cu") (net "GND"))
 (segment (start 144.9435 82.8863) (end 144.8933 82.8361) (width 0.2) (layer "B.Cu") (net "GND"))
 (segment (start 127.501 76.9) (end 127.501 79.8826) (width 0.15) (layer "B.Cu") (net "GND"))
 (segment (start 144.9435 84.9315) (end 144.9435 82.8863) (width 0.2) (layer "B.Cu") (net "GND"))
 (segment (start 127.5 76.9) (end 127.501 76.9) (width 0.2) (layer "B.Cu") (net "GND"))
 (segment (start 130.1467 82.5283) (end 126.525 86.15) (width 0.2) (layer "B.Cu") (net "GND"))
 (segment (start 134.0387 82.8361) (end 132.2466 84.6282) (width 0.2) (layer "B.Cu") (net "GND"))
 (segment (start 127.501 79.8826) (end 109.1562 79.8826) (width 0.2) (layer "B.Cu") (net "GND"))
 (segment (start 130.1467 82.5283) (end 132.2466 84.6282) (width 0.15) (layer "B.Cu") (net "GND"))
 (segment (start 144.8933 82.8361) (end 147 80.7294) (width 0.2) (layer "B.Cu") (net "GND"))
 (segment (start 109.1562 79.8826) (end 109.1562 85.1188) (width 0.2) (layer "B.Cu") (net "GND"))
 (segment (start 151.1575 39.98) (end 144.8075 46.33) (width 0.2) (layer "B.Cu") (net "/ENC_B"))
 (segment (start 116.9915 56.1017) (end 105.0017 56.1017) (width 0.2) (layer "B.Cu") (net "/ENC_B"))
 (segment (start 144.8075 46.33) (end 126.7632 46.33) (width 0.2) (layer "B.Cu") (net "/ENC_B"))
 (segment (start 126.7632 46.33) (end 116.9915 56.1017) (width 0.2) (layer "B.Cu") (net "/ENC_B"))
 (segment (start 105.0017 56.1017) (end 100.6 51.7) (width 0.2) (layer "B.Cu") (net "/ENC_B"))
 (segment (start 147.5475 41.05) (end 151.1575 37.44) (width 0.2) (layer "B.Cu") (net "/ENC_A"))
 (segment (start 100.6 46.7) (end 101.9017 46.7) (width 0.2) (layer "B.Cu") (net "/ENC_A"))
 (segment (start 103.2034 45.3983) (end 130.0251 45.3983) (width 0.2) (layer "B.Cu") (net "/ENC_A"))
 (segment (start 101.9017 46.7) (end 103.2034 45.3983) (width 0.2) (layer "B.Cu") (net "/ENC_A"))
 (segment (start 130.0251 45.3983) (end 134.3734 41.05) (width 0.2) (layer "B.Cu") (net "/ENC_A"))
 (segment (start 134.3734 41.05) (end 147.5475 41.05) (width 0.2) (layer "B.Cu") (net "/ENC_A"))
 (segment (start 122.1467 87.3226) (end 121.075 86.2509) (width 0.2) (layer "B.Cu") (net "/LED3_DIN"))
 (segment (start 134.5184 83.2757) (end 130.4715 87.3226) (width 0.2) (layer "B.Cu") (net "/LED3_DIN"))
 (segment (start 143.925 84.3324) (end 142.8683 83.2757) (width 0.2) (layer "B.Cu") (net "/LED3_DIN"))
 (segment (start 142.8683 83.2757) (end 134.5184 83.2757) (width 0.2) (layer "B.Cu") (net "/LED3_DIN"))
 (segment (start 130.4715 87.3226) (end 122.1467 87.3226) (width 0.2) (layer "B.Cu") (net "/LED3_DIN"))
 (segment (start 121.075 86.2509) (end 121.075 86.15) (width 0.2) (layer "B.Cu") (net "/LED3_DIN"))
 (segment (start 143.925 84.45) (end 143.925 84.3324) (width 0.2) (layer "B.Cu") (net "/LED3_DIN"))
 (segment (start 126.525 84.4858) (end 126.525 84.65) (width 0.2) (layer "B.Cu") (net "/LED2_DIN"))
 (segment (start 102.675 86.3178) (end 103.6888 87.3316) (width 0.2) (layer "B.Cu") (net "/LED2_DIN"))
 (segment (start 115.4158 87.3316) (end 119.2862 83.4612) (width 0.2) (layer "B.Cu") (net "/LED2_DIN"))
 (segment (start 102.675 86.15) (end 102.675 86.3178) (width 0.2) (layer "B.Cu") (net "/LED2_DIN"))
 (segment (start 119.2862 83.4612) (end 125.5004 83.4612) (width 0.2) (layer "B.Cu") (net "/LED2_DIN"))
 (segment (start 125.5004 83.4612) (end 126.525 84.4858) (width 0.2) (layer "B.Cu") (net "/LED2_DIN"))
 (segment (start 103.6888 87.3316) (end 115.4158 87.3316) (width 0.2) (layer "B.Cu") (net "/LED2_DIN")))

